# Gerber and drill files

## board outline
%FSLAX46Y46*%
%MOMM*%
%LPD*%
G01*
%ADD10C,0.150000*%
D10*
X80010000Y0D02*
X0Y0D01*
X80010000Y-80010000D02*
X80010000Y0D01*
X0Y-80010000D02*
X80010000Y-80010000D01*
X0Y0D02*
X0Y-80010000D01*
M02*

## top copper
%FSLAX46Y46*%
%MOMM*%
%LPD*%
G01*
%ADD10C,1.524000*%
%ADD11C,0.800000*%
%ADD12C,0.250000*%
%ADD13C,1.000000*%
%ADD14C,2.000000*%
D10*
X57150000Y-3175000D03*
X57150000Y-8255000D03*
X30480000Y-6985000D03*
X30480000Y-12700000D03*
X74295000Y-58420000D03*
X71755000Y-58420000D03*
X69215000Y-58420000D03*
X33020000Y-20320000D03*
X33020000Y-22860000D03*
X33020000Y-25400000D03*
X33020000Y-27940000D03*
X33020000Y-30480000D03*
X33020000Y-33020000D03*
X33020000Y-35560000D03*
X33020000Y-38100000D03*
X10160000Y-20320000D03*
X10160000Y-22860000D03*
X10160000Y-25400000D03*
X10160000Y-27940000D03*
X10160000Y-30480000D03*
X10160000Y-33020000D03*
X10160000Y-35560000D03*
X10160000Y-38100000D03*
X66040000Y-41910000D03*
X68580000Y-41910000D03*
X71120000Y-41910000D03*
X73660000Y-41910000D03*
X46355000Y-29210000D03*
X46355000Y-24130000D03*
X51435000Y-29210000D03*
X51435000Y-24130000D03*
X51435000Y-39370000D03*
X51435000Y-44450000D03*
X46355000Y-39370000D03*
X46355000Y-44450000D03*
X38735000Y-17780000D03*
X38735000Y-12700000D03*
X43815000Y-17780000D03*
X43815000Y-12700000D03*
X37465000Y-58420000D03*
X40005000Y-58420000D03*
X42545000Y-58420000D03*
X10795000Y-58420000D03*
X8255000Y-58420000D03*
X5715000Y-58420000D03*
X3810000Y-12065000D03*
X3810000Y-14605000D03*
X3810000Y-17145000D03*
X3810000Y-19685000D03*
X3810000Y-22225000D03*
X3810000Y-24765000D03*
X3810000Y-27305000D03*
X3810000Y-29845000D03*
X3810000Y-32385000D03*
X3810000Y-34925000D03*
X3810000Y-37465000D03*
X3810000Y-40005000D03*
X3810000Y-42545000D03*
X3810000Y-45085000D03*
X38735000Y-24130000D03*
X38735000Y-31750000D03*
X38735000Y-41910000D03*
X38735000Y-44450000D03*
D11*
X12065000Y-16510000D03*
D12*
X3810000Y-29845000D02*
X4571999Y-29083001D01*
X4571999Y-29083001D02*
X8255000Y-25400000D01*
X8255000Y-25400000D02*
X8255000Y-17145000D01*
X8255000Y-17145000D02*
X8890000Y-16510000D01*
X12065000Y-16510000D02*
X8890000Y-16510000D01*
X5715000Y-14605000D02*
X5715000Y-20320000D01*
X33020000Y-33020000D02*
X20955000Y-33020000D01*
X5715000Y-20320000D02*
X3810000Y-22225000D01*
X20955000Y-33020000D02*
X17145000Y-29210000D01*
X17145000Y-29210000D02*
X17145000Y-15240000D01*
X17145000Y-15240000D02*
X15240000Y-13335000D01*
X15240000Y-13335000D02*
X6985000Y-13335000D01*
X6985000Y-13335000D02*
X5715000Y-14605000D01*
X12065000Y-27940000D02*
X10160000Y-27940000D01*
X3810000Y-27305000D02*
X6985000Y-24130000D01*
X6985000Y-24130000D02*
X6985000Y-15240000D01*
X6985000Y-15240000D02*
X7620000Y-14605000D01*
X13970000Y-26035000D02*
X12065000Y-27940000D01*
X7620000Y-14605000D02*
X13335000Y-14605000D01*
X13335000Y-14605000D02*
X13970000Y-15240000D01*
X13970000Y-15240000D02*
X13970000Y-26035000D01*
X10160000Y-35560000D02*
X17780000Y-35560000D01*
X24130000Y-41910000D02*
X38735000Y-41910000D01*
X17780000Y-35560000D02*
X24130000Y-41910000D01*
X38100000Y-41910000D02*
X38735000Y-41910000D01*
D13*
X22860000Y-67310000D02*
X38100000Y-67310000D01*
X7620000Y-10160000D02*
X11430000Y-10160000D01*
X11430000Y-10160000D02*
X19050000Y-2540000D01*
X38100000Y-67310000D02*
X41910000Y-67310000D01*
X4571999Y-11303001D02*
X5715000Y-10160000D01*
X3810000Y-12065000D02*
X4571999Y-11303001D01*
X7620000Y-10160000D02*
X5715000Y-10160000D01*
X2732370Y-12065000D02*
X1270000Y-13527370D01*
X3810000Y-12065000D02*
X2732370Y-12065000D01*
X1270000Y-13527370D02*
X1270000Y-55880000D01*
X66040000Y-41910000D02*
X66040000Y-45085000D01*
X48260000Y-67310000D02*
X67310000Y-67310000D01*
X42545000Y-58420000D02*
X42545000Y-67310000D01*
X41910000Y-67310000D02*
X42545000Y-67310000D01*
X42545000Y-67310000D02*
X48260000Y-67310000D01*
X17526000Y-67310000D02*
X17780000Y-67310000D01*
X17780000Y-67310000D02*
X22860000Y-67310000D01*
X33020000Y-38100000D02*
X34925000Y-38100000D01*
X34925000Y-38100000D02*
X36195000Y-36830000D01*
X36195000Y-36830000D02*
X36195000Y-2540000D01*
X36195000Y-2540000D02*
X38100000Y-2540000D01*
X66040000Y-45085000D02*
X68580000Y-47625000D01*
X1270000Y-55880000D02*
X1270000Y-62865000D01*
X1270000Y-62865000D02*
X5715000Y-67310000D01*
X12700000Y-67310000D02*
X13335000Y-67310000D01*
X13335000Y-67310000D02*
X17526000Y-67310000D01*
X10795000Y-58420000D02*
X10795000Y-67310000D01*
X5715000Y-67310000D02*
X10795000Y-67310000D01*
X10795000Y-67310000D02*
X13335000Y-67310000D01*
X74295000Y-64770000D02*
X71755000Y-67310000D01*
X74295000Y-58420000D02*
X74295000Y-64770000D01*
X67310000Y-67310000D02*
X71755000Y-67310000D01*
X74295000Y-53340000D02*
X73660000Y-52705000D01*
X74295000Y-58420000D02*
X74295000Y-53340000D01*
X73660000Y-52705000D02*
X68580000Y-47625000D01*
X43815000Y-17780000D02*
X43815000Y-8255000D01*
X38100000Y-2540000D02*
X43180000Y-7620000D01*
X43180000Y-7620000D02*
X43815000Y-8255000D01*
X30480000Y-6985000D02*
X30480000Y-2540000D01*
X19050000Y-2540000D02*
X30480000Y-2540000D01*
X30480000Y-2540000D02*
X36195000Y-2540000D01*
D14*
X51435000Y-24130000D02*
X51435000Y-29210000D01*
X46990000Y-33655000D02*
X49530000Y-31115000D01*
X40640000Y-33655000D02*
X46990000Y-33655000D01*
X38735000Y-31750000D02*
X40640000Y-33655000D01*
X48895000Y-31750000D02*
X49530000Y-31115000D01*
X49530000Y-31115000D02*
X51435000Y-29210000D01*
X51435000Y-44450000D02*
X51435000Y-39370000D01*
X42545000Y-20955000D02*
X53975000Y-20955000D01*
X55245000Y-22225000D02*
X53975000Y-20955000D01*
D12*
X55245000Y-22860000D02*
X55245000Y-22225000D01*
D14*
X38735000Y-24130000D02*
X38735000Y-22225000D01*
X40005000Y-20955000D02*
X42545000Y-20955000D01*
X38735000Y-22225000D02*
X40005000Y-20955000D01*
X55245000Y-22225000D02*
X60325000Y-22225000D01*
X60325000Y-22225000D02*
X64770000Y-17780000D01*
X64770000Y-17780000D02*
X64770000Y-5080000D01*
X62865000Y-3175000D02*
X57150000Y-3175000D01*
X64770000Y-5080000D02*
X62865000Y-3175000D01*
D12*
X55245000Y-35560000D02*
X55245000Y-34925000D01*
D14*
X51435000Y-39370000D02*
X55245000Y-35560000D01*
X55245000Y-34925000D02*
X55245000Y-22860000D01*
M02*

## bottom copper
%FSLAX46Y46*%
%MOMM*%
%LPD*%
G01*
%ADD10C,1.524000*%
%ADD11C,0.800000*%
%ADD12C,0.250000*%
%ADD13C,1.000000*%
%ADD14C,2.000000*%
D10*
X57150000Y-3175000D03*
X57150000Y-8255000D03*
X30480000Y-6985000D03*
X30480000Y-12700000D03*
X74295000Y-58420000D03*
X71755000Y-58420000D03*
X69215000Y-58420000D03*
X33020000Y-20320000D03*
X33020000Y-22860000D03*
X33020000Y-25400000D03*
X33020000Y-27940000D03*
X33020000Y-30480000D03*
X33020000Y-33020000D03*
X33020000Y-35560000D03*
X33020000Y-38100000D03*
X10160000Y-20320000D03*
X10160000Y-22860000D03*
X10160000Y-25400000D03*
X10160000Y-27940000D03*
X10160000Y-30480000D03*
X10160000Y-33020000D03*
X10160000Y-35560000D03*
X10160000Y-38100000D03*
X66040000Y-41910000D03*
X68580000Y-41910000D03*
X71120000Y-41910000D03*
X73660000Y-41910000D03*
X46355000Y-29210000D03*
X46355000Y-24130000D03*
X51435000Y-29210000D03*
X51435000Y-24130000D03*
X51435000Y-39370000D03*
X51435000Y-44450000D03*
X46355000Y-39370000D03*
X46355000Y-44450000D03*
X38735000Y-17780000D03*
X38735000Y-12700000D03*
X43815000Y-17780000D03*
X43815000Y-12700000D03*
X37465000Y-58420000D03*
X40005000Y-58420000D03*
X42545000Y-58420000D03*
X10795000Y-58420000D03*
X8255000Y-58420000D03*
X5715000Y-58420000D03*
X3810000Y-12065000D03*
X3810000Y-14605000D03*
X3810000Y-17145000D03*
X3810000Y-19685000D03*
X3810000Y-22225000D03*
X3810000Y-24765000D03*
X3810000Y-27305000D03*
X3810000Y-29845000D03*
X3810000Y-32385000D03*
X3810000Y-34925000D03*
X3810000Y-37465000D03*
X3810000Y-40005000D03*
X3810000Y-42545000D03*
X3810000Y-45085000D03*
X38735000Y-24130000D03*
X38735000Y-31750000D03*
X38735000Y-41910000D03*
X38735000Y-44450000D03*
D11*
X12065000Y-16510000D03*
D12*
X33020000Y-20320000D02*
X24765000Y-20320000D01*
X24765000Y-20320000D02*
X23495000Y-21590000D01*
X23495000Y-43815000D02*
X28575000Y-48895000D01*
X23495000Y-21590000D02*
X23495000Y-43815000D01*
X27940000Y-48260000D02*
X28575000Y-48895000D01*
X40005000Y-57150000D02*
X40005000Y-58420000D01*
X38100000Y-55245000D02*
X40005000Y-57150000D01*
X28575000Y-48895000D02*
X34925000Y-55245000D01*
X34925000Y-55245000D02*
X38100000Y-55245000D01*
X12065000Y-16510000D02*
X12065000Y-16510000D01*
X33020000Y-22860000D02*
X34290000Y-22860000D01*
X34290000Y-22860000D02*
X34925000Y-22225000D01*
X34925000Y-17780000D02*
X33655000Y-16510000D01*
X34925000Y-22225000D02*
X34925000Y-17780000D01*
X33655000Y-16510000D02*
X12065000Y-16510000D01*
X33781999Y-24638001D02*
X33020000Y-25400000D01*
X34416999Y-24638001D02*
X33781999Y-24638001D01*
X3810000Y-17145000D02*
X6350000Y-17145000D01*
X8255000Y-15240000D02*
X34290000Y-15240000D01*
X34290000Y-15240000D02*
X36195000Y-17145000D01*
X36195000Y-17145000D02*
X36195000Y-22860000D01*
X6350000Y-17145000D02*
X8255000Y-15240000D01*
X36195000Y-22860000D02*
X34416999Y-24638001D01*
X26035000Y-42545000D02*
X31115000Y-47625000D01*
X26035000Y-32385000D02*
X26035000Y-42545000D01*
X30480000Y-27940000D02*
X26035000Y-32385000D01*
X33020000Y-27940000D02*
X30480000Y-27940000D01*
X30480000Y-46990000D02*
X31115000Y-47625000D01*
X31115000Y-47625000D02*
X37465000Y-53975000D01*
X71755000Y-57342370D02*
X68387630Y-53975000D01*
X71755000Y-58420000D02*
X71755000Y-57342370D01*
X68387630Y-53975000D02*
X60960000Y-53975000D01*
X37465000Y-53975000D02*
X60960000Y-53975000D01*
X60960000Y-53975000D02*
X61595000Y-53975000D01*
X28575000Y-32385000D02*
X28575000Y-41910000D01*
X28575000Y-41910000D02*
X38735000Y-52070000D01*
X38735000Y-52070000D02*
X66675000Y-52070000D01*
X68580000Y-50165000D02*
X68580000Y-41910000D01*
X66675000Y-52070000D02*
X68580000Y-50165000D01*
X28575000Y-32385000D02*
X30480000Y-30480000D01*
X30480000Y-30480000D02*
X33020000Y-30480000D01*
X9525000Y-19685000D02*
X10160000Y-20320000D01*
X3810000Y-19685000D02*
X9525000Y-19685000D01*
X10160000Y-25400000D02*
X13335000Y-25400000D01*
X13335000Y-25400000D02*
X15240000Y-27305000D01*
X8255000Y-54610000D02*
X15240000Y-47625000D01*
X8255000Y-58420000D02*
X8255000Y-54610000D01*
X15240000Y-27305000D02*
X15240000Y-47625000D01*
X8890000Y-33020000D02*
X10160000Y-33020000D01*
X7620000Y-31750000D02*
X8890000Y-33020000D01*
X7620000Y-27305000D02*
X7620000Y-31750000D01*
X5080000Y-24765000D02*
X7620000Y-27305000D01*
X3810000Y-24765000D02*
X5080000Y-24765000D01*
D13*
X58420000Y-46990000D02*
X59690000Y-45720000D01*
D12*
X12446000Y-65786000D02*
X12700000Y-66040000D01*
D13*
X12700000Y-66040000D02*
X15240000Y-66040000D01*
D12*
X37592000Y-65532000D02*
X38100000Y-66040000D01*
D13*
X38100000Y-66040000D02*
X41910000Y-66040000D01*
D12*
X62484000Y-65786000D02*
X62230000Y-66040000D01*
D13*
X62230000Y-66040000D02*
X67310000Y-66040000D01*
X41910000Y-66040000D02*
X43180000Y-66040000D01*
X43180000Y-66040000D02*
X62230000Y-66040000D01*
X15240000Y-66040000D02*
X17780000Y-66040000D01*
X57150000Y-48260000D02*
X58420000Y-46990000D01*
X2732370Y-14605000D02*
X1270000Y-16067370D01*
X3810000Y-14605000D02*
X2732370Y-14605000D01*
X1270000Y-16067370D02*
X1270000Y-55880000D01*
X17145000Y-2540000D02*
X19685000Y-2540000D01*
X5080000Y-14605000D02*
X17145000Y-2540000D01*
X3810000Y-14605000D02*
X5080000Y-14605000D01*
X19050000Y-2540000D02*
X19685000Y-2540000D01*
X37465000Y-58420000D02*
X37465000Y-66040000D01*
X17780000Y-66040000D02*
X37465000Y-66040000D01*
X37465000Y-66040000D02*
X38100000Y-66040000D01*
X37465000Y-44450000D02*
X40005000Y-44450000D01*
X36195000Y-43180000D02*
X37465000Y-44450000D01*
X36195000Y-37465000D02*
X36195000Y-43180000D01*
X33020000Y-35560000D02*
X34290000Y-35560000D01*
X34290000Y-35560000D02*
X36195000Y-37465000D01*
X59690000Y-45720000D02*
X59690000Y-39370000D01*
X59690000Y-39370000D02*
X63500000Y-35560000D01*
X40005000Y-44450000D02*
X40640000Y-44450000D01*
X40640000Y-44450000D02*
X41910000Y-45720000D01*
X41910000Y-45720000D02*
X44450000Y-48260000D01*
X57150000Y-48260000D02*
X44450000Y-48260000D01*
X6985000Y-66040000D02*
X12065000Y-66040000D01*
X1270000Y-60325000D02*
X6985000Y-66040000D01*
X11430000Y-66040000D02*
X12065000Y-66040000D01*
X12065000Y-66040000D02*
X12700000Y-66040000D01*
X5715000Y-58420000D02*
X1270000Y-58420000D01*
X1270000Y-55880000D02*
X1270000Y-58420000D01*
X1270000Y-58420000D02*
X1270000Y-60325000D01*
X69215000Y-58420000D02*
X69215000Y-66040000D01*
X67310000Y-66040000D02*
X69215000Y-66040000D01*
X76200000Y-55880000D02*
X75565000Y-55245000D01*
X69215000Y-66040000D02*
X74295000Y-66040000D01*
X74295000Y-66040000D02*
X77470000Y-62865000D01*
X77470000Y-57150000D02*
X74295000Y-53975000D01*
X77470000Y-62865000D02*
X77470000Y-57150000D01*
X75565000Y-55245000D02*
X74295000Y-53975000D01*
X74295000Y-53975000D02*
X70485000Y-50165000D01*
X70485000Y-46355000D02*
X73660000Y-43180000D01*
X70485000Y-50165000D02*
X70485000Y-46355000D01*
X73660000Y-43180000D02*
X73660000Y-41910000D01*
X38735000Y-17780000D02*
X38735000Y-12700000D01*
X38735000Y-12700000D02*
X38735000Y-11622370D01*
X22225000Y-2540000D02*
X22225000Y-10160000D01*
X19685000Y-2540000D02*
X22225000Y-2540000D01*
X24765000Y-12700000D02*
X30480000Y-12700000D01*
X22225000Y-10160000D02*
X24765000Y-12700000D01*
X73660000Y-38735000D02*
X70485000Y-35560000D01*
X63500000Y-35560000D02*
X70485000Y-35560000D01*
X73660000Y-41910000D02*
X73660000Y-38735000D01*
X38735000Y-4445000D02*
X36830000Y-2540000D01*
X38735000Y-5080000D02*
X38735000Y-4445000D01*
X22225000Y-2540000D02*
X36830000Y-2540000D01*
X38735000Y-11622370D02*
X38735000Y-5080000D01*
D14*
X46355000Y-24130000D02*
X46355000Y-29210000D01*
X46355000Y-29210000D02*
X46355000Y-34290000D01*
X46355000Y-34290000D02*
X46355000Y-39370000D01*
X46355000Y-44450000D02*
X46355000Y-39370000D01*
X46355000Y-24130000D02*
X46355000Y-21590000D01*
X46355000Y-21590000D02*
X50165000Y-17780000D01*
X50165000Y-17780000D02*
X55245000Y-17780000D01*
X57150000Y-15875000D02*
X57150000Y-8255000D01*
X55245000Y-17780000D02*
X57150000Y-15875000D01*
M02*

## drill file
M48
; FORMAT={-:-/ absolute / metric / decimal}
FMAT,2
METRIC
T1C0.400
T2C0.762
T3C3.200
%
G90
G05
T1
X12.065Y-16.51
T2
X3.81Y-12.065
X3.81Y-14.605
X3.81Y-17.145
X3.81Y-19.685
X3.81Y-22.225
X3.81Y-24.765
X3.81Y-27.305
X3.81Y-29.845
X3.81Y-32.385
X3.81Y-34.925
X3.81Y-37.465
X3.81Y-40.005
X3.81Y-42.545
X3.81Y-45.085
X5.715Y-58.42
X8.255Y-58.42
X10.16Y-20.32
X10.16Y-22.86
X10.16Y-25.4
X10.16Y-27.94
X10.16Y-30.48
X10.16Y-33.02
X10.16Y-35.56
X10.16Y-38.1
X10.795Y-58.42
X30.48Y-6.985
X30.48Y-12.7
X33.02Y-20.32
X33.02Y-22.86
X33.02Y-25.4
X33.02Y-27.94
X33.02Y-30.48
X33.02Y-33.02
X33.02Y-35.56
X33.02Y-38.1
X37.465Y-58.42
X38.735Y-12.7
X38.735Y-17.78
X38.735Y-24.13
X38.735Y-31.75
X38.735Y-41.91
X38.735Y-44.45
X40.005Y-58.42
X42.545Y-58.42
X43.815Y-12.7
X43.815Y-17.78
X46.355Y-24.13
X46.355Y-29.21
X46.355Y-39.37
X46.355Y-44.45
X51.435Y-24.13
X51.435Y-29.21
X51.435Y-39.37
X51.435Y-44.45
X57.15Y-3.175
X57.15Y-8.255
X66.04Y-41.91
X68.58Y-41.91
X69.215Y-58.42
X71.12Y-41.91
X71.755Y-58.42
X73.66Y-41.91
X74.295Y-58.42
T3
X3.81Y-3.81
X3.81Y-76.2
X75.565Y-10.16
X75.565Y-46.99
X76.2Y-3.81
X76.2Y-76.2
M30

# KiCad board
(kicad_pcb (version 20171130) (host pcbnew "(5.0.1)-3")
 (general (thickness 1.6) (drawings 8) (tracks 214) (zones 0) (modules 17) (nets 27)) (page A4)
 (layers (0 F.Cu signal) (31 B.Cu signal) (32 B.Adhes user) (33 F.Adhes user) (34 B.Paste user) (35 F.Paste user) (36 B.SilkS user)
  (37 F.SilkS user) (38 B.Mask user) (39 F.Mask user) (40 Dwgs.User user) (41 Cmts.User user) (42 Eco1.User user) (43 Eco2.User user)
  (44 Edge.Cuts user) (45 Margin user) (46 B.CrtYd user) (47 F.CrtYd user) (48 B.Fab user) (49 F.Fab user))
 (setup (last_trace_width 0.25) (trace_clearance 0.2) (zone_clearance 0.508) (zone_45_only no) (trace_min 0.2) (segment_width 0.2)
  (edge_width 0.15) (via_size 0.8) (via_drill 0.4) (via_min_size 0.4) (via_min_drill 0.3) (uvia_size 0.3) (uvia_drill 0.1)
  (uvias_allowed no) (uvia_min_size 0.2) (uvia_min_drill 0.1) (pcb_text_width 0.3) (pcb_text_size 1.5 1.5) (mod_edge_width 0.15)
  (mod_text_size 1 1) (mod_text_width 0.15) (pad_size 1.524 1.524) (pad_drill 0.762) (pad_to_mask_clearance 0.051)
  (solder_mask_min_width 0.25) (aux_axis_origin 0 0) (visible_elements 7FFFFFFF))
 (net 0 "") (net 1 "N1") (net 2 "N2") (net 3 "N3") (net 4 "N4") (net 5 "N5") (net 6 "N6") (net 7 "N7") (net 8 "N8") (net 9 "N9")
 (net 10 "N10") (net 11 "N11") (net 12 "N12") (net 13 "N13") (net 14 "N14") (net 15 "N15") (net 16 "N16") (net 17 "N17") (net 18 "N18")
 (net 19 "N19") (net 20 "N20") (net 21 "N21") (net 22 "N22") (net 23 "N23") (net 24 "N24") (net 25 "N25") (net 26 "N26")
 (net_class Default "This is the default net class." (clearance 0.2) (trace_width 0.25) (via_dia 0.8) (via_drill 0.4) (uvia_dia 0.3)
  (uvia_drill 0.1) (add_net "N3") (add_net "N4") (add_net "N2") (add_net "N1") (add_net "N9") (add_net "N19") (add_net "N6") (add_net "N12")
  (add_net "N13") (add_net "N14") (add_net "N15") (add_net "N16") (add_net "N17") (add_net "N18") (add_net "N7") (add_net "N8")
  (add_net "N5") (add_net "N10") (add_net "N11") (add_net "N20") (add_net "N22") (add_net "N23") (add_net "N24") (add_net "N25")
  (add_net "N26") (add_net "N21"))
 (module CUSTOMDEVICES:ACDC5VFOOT (layer F.Cu) (at 58.42 0 270)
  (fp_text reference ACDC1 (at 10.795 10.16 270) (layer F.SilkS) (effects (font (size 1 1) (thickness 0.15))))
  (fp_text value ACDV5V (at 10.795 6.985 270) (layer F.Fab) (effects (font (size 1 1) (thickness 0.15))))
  (pad 2 thru_hole circle (at 3.175 1.27 270) (size 1.524 1.524) (drill 0.762) (layers *.Cu *.Mask) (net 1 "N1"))
  (pad 1 thru_hole circle (at 8.255 1.27 270) (size 1.524 1.524) (drill 0.762) (layers *.Cu *.Mask) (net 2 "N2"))
  (pad 4 thru_hole circle (at 6.985 27.94 270) (size 1.524 1.524) (drill 0.762) (layers *.Cu *.Mask) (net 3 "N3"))
  (pad 3 thru_hole circle (at 12.7 27.94 270) (size 1.524 1.524) (drill 0.762) (layers *.Cu *.Mask) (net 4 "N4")))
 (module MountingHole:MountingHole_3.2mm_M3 (layer F.Cu) (at 75.565 46.99)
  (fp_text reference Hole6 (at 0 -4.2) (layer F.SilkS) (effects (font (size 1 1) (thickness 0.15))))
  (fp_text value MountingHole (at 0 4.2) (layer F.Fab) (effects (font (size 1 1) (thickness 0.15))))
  (pad 1 np_thru_hole circle (at 0 0) (size 3.2 3.2) (drill 3.2) (layers *.Cu *.Mask)))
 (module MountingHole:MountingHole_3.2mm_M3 (layer F.Cu) (at 75.565 10.16)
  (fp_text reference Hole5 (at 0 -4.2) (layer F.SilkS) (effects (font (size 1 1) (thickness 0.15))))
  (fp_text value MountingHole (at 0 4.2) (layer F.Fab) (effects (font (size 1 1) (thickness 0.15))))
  (pad 1 np_thru_hole circle (at 0 0) (size 3.2 3.2) (drill 3.2) (layers *.Cu *.Mask)))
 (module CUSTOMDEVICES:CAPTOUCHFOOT (layer F.Cu) (at 71.755 63.5 180)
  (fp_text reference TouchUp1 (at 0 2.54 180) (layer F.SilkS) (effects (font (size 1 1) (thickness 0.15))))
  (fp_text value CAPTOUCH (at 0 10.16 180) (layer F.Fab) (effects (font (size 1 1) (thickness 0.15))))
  (pad 1 thru_hole circle (at -2.54 5.08 180) (size 1.524 1.524) (drill 0.762) (layers *.Cu *.Mask) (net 3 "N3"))
  (pad 2 thru_hole circle (at 0 5.08 180) (size 1.524 1.524) (drill 0.762) (layers *.Cu *.Mask) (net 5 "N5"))
  (pad 3 thru_hole circle (at 2.54 5.08 180) (size 1.524 1.524) (drill 0.762) (layers *.Cu *.Mask) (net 4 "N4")))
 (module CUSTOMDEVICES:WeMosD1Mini (layer F.Cu) (at 21.59 30.48)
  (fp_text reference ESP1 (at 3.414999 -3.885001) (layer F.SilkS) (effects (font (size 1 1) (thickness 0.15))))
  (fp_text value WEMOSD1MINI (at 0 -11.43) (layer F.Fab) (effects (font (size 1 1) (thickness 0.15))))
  (pad 1 thru_hole circle (at 11.43 -10.16) (size 1.524 1.524) (drill 0.762) (layers *.Cu *.Mask) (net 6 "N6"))
  (pad 2 thru_hole circle (at 11.43 -7.62) (size 1.524 1.524) (drill 0.762) (layers *.Cu *.Mask) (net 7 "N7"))
  (pad 3 thru_hole circle (at 11.43 -5.08) (size 1.524 1.524) (drill 0.762) (layers *.Cu *.Mask) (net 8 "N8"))
  (pad 4 thru_hole circle (at 11.43 -2.54) (size 1.524 1.524) (drill 0.762) (layers *.Cu *.Mask) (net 5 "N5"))
  (pad 5 thru_hole circle (at 11.43 0) (size 1.524 1.524) (drill 0.762) (layers *.Cu *.Mask) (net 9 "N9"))
  (pad 6 thru_hole circle (at 11.43 2.54) (size 1.524 1.524) (drill 0.762) (layers *.Cu *.Mask) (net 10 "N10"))
  (pad 7 thru_hole circle (at 11.43 5.08) (size 1.524 1.524) (drill 0.762) (layers *.Cu *.Mask) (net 4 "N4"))
  (pad 8 thru_hole circle (at 11.43 7.62) (size 1.524 1.524) (drill 0.762) (layers *.Cu *.Mask) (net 3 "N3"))
  (pad 9 thru_hole circle (at -11.43 -10.16) (size 1.524 1.524) (drill 0.762) (layers *.Cu *.Mask) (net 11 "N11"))
  (pad 10 thru_hole circle (at -11.43 -7.62) (size 1.524 1.524) (drill 0.762) (layers *.Cu *.Mask) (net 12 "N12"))
  (pad 11 thru_hole circle (at -11.43 -5.08) (size 1.524 1.524) (drill 0.762) (layers *.Cu *.Mask) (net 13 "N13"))
  (pad 12 thru_hole circle (at -11.43 -2.54) (size 1.524 1.524) (drill 0.762) (layers *.Cu *.Mask) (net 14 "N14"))
  (pad 13 thru_hole circle (at -11.43 0) (size 1.524 1.524) (drill 0.762) (layers *.Cu *.Mask) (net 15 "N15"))
  (pad 14 thru_hole circle (at -11.43 2.54) (size 1.524 1.524) (drill 0.762) (layers *.Cu *.Mask) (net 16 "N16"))
  (pad 15 thru_hole circle (at -11.43 5.08) (size 1.524 1.524) (drill 0.762) (layers *.Cu *.Mask) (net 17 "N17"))
  (pad 16 thru_hole circle (at -11.43 7.62) (size 1.524 1.524) (drill 0.762) (layers *.Cu *.Mask) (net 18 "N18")))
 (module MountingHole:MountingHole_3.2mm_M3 (layer F.Cu) (at 76.2 76.2)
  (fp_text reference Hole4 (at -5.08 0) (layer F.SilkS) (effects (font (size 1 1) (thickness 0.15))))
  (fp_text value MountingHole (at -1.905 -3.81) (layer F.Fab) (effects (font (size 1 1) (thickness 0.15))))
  (pad 1 np_thru_hole circle (at 0 0) (size 3.2 3.2) (drill 3.2) (layers *.Cu *.Mask)))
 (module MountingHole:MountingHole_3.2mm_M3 (layer F.Cu) (at 3.81 76.2)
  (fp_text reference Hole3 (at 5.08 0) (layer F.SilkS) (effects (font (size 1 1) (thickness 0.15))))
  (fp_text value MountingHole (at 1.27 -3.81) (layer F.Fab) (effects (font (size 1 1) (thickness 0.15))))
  (pad 1 np_thru_hole circle (at 0 0) (size 3.2 3.2) (drill 3.2) (layers *.Cu *.Mask)))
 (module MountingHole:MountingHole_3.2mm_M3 (layer F.Cu) (at 76.2 3.81)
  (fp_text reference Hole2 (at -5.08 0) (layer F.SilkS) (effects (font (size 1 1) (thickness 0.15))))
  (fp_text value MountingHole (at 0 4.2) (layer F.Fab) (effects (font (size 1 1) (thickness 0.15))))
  (pad 1 np_thru_hole circle (at 0 0) (size 3.2 3.2) (drill 3.2) (layers *.Cu *.Mask)))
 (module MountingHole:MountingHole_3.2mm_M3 (layer F.Cu) (at 3.81 3.81)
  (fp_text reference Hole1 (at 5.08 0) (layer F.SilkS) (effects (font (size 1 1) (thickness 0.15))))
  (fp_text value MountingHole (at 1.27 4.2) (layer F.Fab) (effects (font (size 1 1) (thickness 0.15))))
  (pad 1 np_thru_hole circle (at 0 0) (size 3.2 3.2) (drill 3.2) (layers *.Cu *.Mask)))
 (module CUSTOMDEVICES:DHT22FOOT (layer F.Cu) (at 71.12 29.21)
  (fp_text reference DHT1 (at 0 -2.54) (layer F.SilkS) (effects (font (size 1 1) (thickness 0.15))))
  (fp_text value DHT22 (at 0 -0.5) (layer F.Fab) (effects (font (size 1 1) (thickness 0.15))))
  (pad 1 thru_hole circle (at -5.08 12.7) (size 1.524 1.524) (drill 0.762) (layers *.Cu *.Mask) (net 3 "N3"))
  (pad 2 thru_hole circle (at -2.54 12.7) (size 1.524 1.524) (drill 0.762) (layers *.Cu *.Mask) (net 9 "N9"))
  (pad 3 thru_hole circle (at 0 12.7) (size 1.524 1.524) (drill 0.762) (layers *.Cu *.Mask) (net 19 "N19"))
  (pad 4 thru_hole circle (at 2.54 12.7) (size 1.524 1.524) (drill 0.762) (layers *.Cu *.Mask) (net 4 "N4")))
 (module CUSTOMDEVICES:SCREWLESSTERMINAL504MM (layer F.Cu) (at 46.355 26.67 180)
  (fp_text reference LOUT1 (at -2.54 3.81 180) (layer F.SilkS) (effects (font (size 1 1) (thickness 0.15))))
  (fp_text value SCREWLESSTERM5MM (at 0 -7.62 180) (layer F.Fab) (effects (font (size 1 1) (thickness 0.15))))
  (pad 2 thru_hole circle (at 0 -2.54 180) (size 1.524 1.524) (drill 0.762) (layers *.Cu *.Mask) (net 2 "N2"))
  (pad 2 thru_hole circle (at 0 2.54 180) (size 1.524 1.524) (drill 0.762) (layers *.Cu *.Mask) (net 2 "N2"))
  (pad 1 thru_hole circle (at -5.08 -2.54 180) (size 1.524 1.524) (drill 0.762) (layers *.Cu *.Mask) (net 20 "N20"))
  (pad 1 thru_hole circle (at -5.08 2.54 180) (size 1.524 1.524) (drill 0.762) (layers *.Cu *.Mask) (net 20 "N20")))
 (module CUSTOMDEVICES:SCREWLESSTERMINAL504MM (layer F.Cu) (at 46.355 41.91 180)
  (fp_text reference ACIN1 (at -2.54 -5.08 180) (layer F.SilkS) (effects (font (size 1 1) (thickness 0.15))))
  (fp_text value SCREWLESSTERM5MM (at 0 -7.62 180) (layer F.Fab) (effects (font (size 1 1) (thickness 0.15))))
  (pad 1 thru_hole circle (at -5.08 2.54 180) (size 1.524 1.524) (drill 0.762) (layers *.Cu *.Mask) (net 1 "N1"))
  (pad 1 thru_hole circle (at -5.08 -2.54 180) (size 1.524 1.524) (drill 0.762) (layers *.Cu *.Mask) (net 1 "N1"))
  (pad 2 thru_hole circle (at 0 2.54 180) (size 1.524 1.524) (drill 0.762) (layers *.Cu *.Mask) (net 2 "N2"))
  (pad 2 thru_hole circle (at 0 -2.54 180) (size 1.524 1.524) (drill 0.762) (layers *.Cu *.Mask) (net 2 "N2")))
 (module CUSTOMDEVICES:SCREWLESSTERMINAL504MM (layer F.Cu) (at 38.735 15.24 180)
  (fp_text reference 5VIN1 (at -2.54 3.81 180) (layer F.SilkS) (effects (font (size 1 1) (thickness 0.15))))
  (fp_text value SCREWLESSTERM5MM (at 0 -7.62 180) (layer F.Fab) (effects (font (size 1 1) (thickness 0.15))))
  (pad 2 thru_hole circle (at 0 -2.54 180) (size 1.524 1.524) (drill 0.762) (layers *.Cu *.Mask) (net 4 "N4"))
  (pad 2 thru_hole circle (at 0 2.54 180) (size 1.524 1.524) (drill 0.762) (layers *.Cu *.Mask) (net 4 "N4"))
  (pad 1 thru_hole circle (at -5.08 -2.54 180) (size 1.524 1.524) (drill 0.762) (layers *.Cu *.Mask) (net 3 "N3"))
  (pad 1 thru_hole circle (at -5.08 2.54 180) (size 1.524 1.524) (drill 0.762) (layers *.Cu *.Mask) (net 3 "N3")))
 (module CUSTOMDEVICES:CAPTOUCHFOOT (layer F.Cu) (at 40.005 63.5 180)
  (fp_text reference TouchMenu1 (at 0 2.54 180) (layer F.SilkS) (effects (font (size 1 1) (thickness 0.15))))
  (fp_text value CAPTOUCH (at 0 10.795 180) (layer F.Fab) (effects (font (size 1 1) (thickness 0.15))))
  (pad 3 thru_hole circle (at 2.54 5.08 180) (size 1.524 1.524) (drill 0.762) (layers *.Cu *.Mask) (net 4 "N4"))
  (pad 2 thru_hole circle (at 0 5.08 180) (size 1.524 1.524) (drill 0.762) (layers *.Cu *.Mask) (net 6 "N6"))
  (pad 1 thru_hole circle (at -2.54 5.08 180) (size 1.524 1.524) (drill 0.762) (layers *.Cu *.Mask) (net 3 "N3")))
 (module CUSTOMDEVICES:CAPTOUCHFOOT (layer F.Cu) (at 8.255 63.5 180)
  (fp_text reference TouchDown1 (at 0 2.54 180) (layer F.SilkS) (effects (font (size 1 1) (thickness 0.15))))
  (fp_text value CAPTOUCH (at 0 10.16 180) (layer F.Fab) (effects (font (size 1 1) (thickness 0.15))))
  (pad 1 thru_hole circle (at -2.54 5.08 180) (size 1.524 1.524) (drill 0.762) (layers *.Cu *.Mask) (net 3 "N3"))
  (pad 2 thru_hole circle (at 0 5.08 180) (size 1.524 1.524) (drill 0.762) (layers *.Cu *.Mask) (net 13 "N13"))
  (pad 3 thru_hole circle (at 2.54 5.08 180) (size 1.524 1.524) (drill 0.762) (layers *.Cu *.Mask) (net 4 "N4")))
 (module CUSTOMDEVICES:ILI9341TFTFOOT (layer F.Cu) (at 6.35 29.845 180)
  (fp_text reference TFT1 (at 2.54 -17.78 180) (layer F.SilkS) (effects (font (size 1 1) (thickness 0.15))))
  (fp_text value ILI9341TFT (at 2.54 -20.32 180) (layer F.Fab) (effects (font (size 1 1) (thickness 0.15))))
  (pad 1 thru_hole circle (at 2.54 17.78 180) (size 1.524 1.524) (drill 0.762) (layers *.Cu *.Mask) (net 3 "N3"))
  (pad 2 thru_hole circle (at 2.54 15.24 180) (size 1.524 1.524) (drill 0.762) (layers *.Cu *.Mask) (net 4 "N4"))
  (pad 3 thru_hole circle (at 2.54 12.7 180) (size 1.524 1.524) (drill 0.762) (layers *.Cu *.Mask) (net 8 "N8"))
  (pad 4 thru_hole circle (at 2.54 10.16 180) (size 1.524 1.524) (drill 0.762) (layers *.Cu *.Mask) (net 11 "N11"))
  (pad 5 thru_hole circle (at 2.54 7.62 180) (size 1.524 1.524) (drill 0.762) (layers *.Cu *.Mask) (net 10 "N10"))
  (pad 6 thru_hole circle (at 2.54 5.08 180) (size 1.524 1.524) (drill 0.762) (layers *.Cu *.Mask) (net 16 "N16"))
  (pad 7 thru_hole circle (at 2.54 2.54 180) (size 1.524 1.524) (drill 0.762) (layers *.Cu *.Mask) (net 14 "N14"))
  (pad 8 thru_hole circle (at 2.54 0 180) (size 1.524 1.524) (drill 0.762) (layers *.Cu *.Mask) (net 7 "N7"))
  (pad 9 thru_hole circle (at 2.54 -2.54 180) (size 1.524 1.524) (drill 0.762) (layers *.Cu *.Mask) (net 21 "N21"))
  (pad 10 thru_hole circle (at 2.54 -5.08 180) (size 1.524 1.524) (drill 0.762) (layers *.Cu *.Mask) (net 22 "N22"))
  (pad 11 thru_hole circle (at 2.54 -7.62 180) (size 1.524 1.524) (drill 0.762) (layers *.Cu *.Mask) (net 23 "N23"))
  (pad 12 thru_hole circle (at 2.54 -10.16 180) (size 1.524 1.524) (drill 0.762) (layers *.Cu *.Mask) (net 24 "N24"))
  (pad 13 thru_hole circle (at 2.54 -12.7 180) (size 1.524 1.524) (drill 0.762) (layers *.Cu *.Mask) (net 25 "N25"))
  (pad 14 thru_hole circle (at 2.54 -15.24 180) (size 1.524 1.524) (drill 0.762) (layers *.Cu *.Mask) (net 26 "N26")))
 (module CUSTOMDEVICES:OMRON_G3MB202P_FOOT (layer F.Cu) (at 38.735 34.29)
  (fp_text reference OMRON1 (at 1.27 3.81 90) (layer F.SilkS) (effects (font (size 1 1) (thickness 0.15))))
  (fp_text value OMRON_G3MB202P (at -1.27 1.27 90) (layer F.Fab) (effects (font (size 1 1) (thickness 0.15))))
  (pad 1 thru_hole circle (at 0 -10.16) (size 1.524 1.524) (drill 0.762) (layers *.Cu *.Mask) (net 1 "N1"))
  (pad 2 thru_hole circle (at 0 -2.54) (size 1.524 1.524) (drill 0.762) (layers *.Cu *.Mask) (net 20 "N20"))
  (pad 3 thru_hole circle (at 0 7.62) (size 1.524 1.524) (drill 0.762) (layers *.Cu *.Mask) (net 17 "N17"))
  (pad 4 thru_hole circle (at 0 10.16) (size 1.524 1.524) (drill 0.762) (layers *.Cu *.Mask) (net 4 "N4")))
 (gr_line (start 80.01 0) (end 0 0) (layer Edge.Cuts) (width 0.15))
 (gr_line (start 80.01 80.01) (end 80.01 0) (layer Edge.Cuts) (width 0.15))
 (gr_line (start 0 80.01) (end 80.01 80.01) (layer Edge.Cuts) (width 0.15))
 (gr_line (start 0 0) (end 0 80.01) (layer Edge.Cuts) (width 0.15))
 (segment (start 33.02 20.32) (end 24.765 20.32) (width 0.25) (layer B.Cu) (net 6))
 (segment (start 24.765 20.32) (end 23.495 21.59) (width 0.25) (layer B.Cu) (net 6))
 (segment (start 23.495 43.815) (end 28.575 48.895) (width 0.25) (layer B.Cu) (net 6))
 (segment (start 23.495 21.59) (end 23.495 43.815) (width 0.25) (layer B.Cu) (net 6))
 (segment (start 27.94 48.26) (end 28.575 48.895) (width 0.25) (layer B.Cu) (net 6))
 (segment (start 40.005 57.15) (end 40.005 58.42) (width 0.25) (layer B.Cu) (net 6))
 (segment (start 38.1 55.245) (end 40.005 57.15) (width 0.25) (layer B.Cu) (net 6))
 (segment (start 28.575 48.895) (end 34.925 55.245) (width 0.25) (layer B.Cu) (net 6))
 (segment (start 34.925 55.245) (end 38.1 55.245) (width 0.25) (layer B.Cu) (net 6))
 (segment (start 3.81 29.845) (end 4.571999 29.083001) (width 0.25) (layer F.Cu) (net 7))
 (segment (start 4.571999 29.083001) (end 8.255 25.4) (width 0.25) (layer F.Cu) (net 7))
 (segment (start 8.255 25.4) (end 8.255 17.145) (width 0.25) (layer F.Cu) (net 7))
 (segment (start 8.255 17.145) (end 8.89 16.51) (width 0.25) (layer F.Cu) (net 7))
 (segment (start 12.065 16.51) (end 12.065 16.51) (width 0.25) (layer B.Cu) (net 7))
 (via (at 12.065 16.51) (size 0.8) (drill 0.4) (layers F.Cu B.Cu) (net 7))
 (segment (start 12.065 16.51) (end 8.89 16.51) (width 0.25) (layer F.Cu) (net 7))
 (segment (start 33.02 22.86) (end 34.29 22.86) (width 0.25) (layer B.Cu) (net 7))
 (segment (start 34.29 22.86) (end 34.925 22.225) (width 0.25) (layer B.Cu) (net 7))
 (segment (start 34.925 17.78) (end 33.655 16.51) (width 0.25) (layer B.Cu) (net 7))
 (segment (start 34.925 22.225) (end 34.925 17.78) (width 0.25) (layer B.Cu) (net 7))
 (segment (start 33.655 16.51) (end 12.065 16.51) (width 0.25) (layer B.Cu) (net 7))
 (segment (start 33.781999 24.638001) (end 33.02 25.4) (width 0.25) (layer B.Cu) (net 8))
 (segment (start 34.416999 24.638001) (end 33.781999 24.638001) (width 0.25) (layer B.Cu) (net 8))
 (segment (start 3.81 17.145) (end 6.35 17.145) (width 0.25) (layer B.Cu) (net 8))
 (segment (start 8.255 15.24) (end 34.29 15.24) (width 0.25) (layer B.Cu) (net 8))
 (segment (start 34.29 15.24) (end 36.195 17.145) (width 0.25) (layer B.Cu) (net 8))
 (segment (start 36.195 17.145) (end 36.195 22.86) (width 0.25) (layer B.Cu) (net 8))
 (segment (start 6.35 17.145) (end 8.255 15.24) (width 0.25) (layer B.Cu) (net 8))
 (segment (start 36.195 22.86) (end 34.416999 24.638001) (width 0.25) (layer B.Cu) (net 8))
 (segment (start 26.035 42.545) (end 31.115 47.625) (width 0.25) (layer B.Cu) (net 5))
 (segment (start 26.035 32.385) (end 26.035 42.545) (width 0.25) (layer B.Cu) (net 5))
 (segment (start 30.48 27.94) (end 26.035 32.385) (width 0.25) (layer B.Cu) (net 5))
 (segment (start 33.02 27.94) (end 30.48 27.94) (width 0.25) (layer B.Cu) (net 5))
 (segment (start 30.48 46.99) (end 31.115 47.625) (width 0.25) (layer B.Cu) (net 5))
 (segment (start 31.115 47.625) (end 37.465 53.975) (width 0.25) (layer B.Cu) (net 5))
 (segment (start 71.755 57.34237) (end 68.38763 53.975) (width 0.25) (layer B.Cu) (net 5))
 (segment (start 71.755 58.42) (end 71.755 57.34237) (width 0.25) (layer B.Cu) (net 5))
 (segment (start 68.38763 53.975) (end 60.96 53.975) (width 0.25) (layer B.Cu) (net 5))
 (segment (start 37.465 53.975) (end 60.96 53.975) (width 0.25) (layer B.Cu) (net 5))
 (segment (start 60.96 53.975) (end 61.595 53.975) (width 0.25) (layer B.Cu) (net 5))
 (segment (start 28.575 32.385) (end 28.575 41.91) (width 0.25) (layer B.Cu) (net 9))
 (segment (start 28.575 41.91) (end 38.735 52.07) (width 0.25) (layer B.Cu) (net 9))
 (segment (start 38.735 52.07) (end 66.675 52.07) (width 0.25) (layer B.Cu) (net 9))
 (segment (start 68.58 50.165) (end 68.58 41.91) (width 0.25) (layer B.Cu) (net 9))
 (segment (start 66.675 52.07) (end 68.58 50.165) (width 0.25) (layer B.Cu) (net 9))
 (segment (start 28.575 32.385) (end 30.48 30.48) (width 0.25) (layer B.Cu) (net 9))
 (segment (start 30.48 30.48) (end 33.02 30.48) (width 0.25) (layer B.Cu) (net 9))
 (segment (start 5.715 14.605) (end 5.715 20.32) (width 0.25) (layer F.Cu) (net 10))
 (segment (start 33.02 33.02) (end 20.955 33.02) (width 0.25) (layer F.Cu) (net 10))
 (segment (start 5.715 20.32) (end 3.81 22.225) (width 0.25) (layer F.Cu) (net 10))
 (segment (start 20.955 33.02) (end 17.145 29.21) (width 0.25) (layer F.Cu) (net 10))
 (segment (start 17.145 29.21) (end 17.145 15.24) (width 0.25) (layer F.Cu) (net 10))
 (segment (start 17.145 15.24) (end 15.24 13.335) (width 0.25) (layer F.Cu) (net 10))
 (segment (start 15.24 13.335) (end 6.985 13.335) (width 0.25) (layer F.Cu) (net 10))
 (segment (start 6.985 13.335) (end 5.715 14.605) (width 0.25) (layer F.Cu) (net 10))
 (segment (start 9.525 19.685) (end 10.16 20.32) (width 0.25) (layer B.Cu) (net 11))
 (segment (start 3.81 19.685) (end 9.525 19.685) (width 0.25) (layer B.Cu) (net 11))
 (segment (start 10.16 25.4) (end 13.335 25.4) (width 0.25) (layer B.Cu) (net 13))
 (segment (start 13.335 25.4) (end 15.24 27.305) (width 0.25) (layer B.Cu) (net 13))
 (segment (start 8.255 54.61) (end 15.24 47.625) (width 0.25) (layer B.Cu) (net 13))
 (segment (start 8.255 58.42) (end 8.255 54.61) (width 0.25) (layer B.Cu) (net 13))
 (segment (start 15.24 27.305) (end 15.24 47.625) (width 0.25) (layer B.Cu) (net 13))
 (segment (start 12.065 27.94) (end 10.16 27.94) (width 0.25) (layer F.Cu) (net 14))
 (segment (start 3.81 27.305) (end 6.985 24.13) (width 0.25) (layer F.Cu) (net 14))
 (segment (start 6.985 24.13) (end 6.985 15.24) (width 0.25) (layer F.Cu) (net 14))
 (segment (start 6.985 15.24) (end 7.62 14.605) (width 0.25) (layer F.Cu) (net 14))
 (segment (start 13.97 26.035) (end 12.065 27.94) (width 0.25) (layer F.Cu) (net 14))
 (segment (start 7.62 14.605) (end 13.335 14.605) (width 0.25) (layer F.Cu) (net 14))
 (segment (start 13.335 14.605) (end 13.97 15.24) (width 0.25) (layer F.Cu) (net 14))
 (segment (start 13.97 15.24) (end 13.97 26.035) (width 0.25) (layer F.Cu) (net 14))
 (segment (start 8.89 33.02) (end 10.16 33.02) (width 0.25) (layer B.Cu) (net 16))
 (segment (start 7.62 31.75) (end 8.89 33.02) (width 0.25) (layer B.Cu) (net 16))
 (segment (start 7.62 27.305) (end 7.62 31.75) (width 0.25) (layer B.Cu) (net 16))
 (segment (start 5.08 24.765) (end 7.62 27.305) (width 0.25) (layer B.Cu) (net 16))
 (segment (start 3.81 24.765) (end 5.08 24.765) (width 0.25) (layer B.Cu) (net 16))
 (segment (start 10.16 35.56) (end 17.78 35.56) (width 0.25) (layer F.Cu) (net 17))
 (segment (start 24.13 41.91) (end 38.735 41.91) (width 0.25) (layer F.Cu) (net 17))
 (segment (start 17.78 35.56) (end 24.13 41.91) (width 0.25) (layer F.Cu) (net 17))
 (segment (start 38.1 41.91) (end 38.735 41.91) (width 0.25) (layer F.Cu) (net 17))
 (segment (start 22.86 67.31) (end 38.1 67.31) (width 1) (layer F.Cu) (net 3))
 (segment (start 7.62 10.16) (end 11.43 10.16) (width 1) (layer F.Cu) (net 3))
 (segment (start 11.43 10.16) (end 19.05 2.54) (width 1) (layer F.Cu) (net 3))
 (segment (start 38.1 67.31) (end 41.91 67.31) (width 1) (layer F.Cu) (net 3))
 (segment (start 4.571999 11.303001) (end 5.715 10.16) (width 1) (layer F.Cu) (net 3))
 (segment (start 3.81 12.065) (end 4.571999 11.303001) (width 1) (layer F.Cu) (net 3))
 (segment (start 7.62 10.16) (end 5.715 10.16) (width 1) (layer F.Cu) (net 3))
 (segment (start 2.73237 12.065) (end 1.27 13.52737) (width 1) (layer F.Cu) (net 3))
 (segment (start 3.81 12.065) (end 2.73237 12.065) (width 1) (layer F.Cu) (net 3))
 (segment (start 1.27 13.52737) (end 1.27 55.88) (width 1) (layer F.Cu) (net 3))
 (segment (start 66.04 41.91) (end 66.04 45.085) (width 1) (layer F.Cu) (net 3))
 (segment (start 48.26 67.31) (end 67.31 67.31) (width 1) (layer F.Cu) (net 3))
 (segment (start 42.545 58.42) (end 42.545 67.31) (width 1) (layer F.Cu) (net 3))
 (segment (start 41.91 67.31) (end 42.545 67.31) (width 1) (layer F.Cu) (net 3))
 (segment (start 42.545 67.31) (end 48.26 67.31) (width 1) (layer F.Cu) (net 3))
 (segment (start 17.526 67.31) (end 17.78 67.31) (width 1) (layer F.Cu) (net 3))
 (segment (start 17.78 67.31) (end 22.86 67.31) (width 1) (layer F.Cu) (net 3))
 (segment (start 33.02 38.1) (end 34.925 38.1) (width 1) (layer F.Cu) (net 3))
 (segment (start 34.925 38.1) (end 36.195 36.83) (width 1) (layer F.Cu) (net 3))
 (segment (start 36.195 36.83) (end 36.195 2.54) (width 1) (layer F.Cu) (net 3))
 (segment (start 36.195 2.54) (end 38.1 2.54) (width 1) (layer F.Cu) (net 3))
 (segment (start 66.04 45.085) (end 68.58 47.625) (width 1) (layer F.Cu) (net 3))
 (segment (start 1.27 55.88) (end 1.27 62.865) (width 1) (layer F.Cu) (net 3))
 (segment (start 1.27 62.865) (end 5.715 67.31) (width 1) (layer F.Cu) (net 3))
 (segment (start 12.7 67.31) (end 13.335 67.31) (width 1) (layer F.Cu) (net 3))
 (segment (start 13.335 67.31) (end 17.526 67.31) (width 1) (layer F.Cu) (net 3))
 (segment (start 10.795 58.42) (end 10.795 67.31) (width 1) (layer F.Cu) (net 3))
 (segment (start 5.715 67.31) (end 10.795 67.31) (width 1) (layer F.Cu) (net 3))
 (segment (start 10.795 67.31) (end 13.335 67.31) (width 1) (layer F.Cu) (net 3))
 (segment (start 74.295 64.77) (end 71.755 67.31) (width 1) (layer F.Cu) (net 3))
 (segment (start 74.295 58.42) (end 74.295 64.77) (width 1) (layer F.Cu) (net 3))
 (segment (start 67.31 67.31) (end 71.755 67.31) (width 1) (layer F.Cu) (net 3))
 (segment (start 74.295 53.34) (end 73.66 52.705) (width 1) (layer F.Cu) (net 3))
 (segment (start 74.295 58.42) (end 74.295 53.34) (width 1) (layer F.Cu) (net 3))
 (segment (start 73.66 52.705) (end 68.58 47.625) (width 1) (layer F.Cu) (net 3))
 (segment (start 43.815 17.78) (end 43.815 8.255) (width 1) (layer F.Cu) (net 3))
 (segment (start 38.1 2.54) (end 43.18 7.62) (width 1) (layer F.Cu) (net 3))
 (segment (start 43.18 7.62) (end 43.815 8.255) (width 1) (layer F.Cu) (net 3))
 (segment (start 30.48 6.985) (end 30.48 2.54) (width 1) (layer F.Cu) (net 3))
 (segment (start 19.05 2.54) (end 30.48 2.54) (width 1) (layer F.Cu) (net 3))
 (segment (start 30.48 2.54) (end 36.195 2.54) (width 1) (layer F.Cu) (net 3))
 (segment (start 58.42 46.99) (end 59.69 45.72) (width 1) (layer B.Cu) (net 4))
 (segment (start 12.446 65.786) (end 12.7 66.04) (width 0.25) (layer B.Cu) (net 4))
 (segment (start 12.7 66.04) (end 15.24 66.04) (width 1) (layer B.Cu) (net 4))
 (segment (start 37.592 65.532) (end 38.1 66.04) (width 0.25) (layer B.Cu) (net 4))
 (segment (start 38.1 66.04) (end 41.91 66.04) (width 1) (layer B.Cu) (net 4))
 (segment (start 62.484 65.786) (end 62.23 66.04) (width 0.25) (layer B.Cu) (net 4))
 (segment (start 62.23 66.04) (end 67.31 66.04) (width 1) (layer B.Cu) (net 4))
 (segment (start 41.91 66.04) (end 43.18 66.04) (width 1) (layer B.Cu) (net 4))
 (segment (start 43.18 66.04) (end 62.23 66.04) (width 1) (layer B.Cu) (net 4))
 (segment (start 15.24 66.04) (end 17.78 66.04) (width 1) (layer B.Cu) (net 4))
 (segment (start 57.15 48.26) (end 58.42 46.99) (width 1) (layer B.Cu) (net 4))
 (segment (start 2.73237 14.605) (end 1.27 16.06737) (width 1) (layer B.Cu) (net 4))
 (segment (start 3.81 14.605) (end 2.73237 14.605) (width 1) (layer B.Cu) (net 4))
 (segment (start 1.27 16.06737) (end 1.27 55.88) (width 1) (layer B.Cu) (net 4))
 (segment (start 17.145 2.54) (end 19.685 2.54) (width 1) (layer B.Cu) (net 4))
 (segment (start 5.08 14.605) (end 17.145 2.54) (width 1) (layer B.Cu) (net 4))
 (segment (start 3.81 14.605) (end 5.08 14.605) (width 1) (layer B.Cu) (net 4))
 (segment (start 19.05 2.54) (end 19.685 2.54) (width 1) (layer B.Cu) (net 4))
 (segment (start 37.465 58.42) (end 37.465 66.04) (width 1) (layer B.Cu) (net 4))
 (segment (start 17.78 66.04) (end 37.465 66.04) (width 1) (layer B.Cu) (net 4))
 (segment (start 37.465 66.04) (end 38.1 66.04) (width 1) (layer B.Cu) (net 4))
 (segment (start 37.465 44.45) (end 40.005 44.45) (width 1) (layer B.Cu) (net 4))
 (segment (start 36.195 43.18) (end 37.465 44.45) (width 1) (layer B.Cu) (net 4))
 (segment (start 36.195 37.465) (end 36.195 43.18) (width 1) (layer B.Cu) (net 4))
 (segment (start 33.02 35.56) (end 34.29 35.56) (width 1) (layer B.Cu) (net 4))
 (segment (start 34.29 35.56) (end 36.195 37.465) (width 1) (layer B.Cu) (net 4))
 (segment (start 59.69 45.72) (end 59.69 39.37) (width 1) (layer B.Cu) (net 4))
 (segment (start 59.69 39.37) (end 63.5 35.56) (width 1) (layer B.Cu) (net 4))
 (segment (start 40.005 44.45) (end 40.64 44.45) (width 1) (layer B.Cu) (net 4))
 (segment (start 40.64 44.45) (end 41.91 45.72) (width 1) (layer B.Cu) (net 4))
 (segment (start 41.91 45.72) (end 44.45 48.26) (width 1) (layer B.Cu) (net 4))
 (segment (start 57.15 48.26) (end 44.45 48.26) (width 1) (layer B.Cu) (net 4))
 (segment (start 6.985 66.04) (end 12.065 66.04) (width 1) (layer B.Cu) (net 4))
 (segment (start 1.27 60.325) (end 6.985 66.04) (width 1) (layer B.Cu) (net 4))
 (segment (start 11.43 66.04) (end 12.065 66.04) (width 1) (layer B.Cu) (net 4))
 (segment (start 12.065 66.04) (end 12.7 66.04) (width 1) (layer B.Cu) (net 4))
 (segment (start 5.715 58.42) (end 1.27 58.42) (width 1) (layer B.Cu) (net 4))
 (segment (start 1.27 55.88) (end 1.27 58.42) (width 1) (layer B.Cu) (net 4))
 (segment (start 1.27 58.42) (end 1.27 60.325) (width 1) (layer B.Cu) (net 4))
 (segment (start 69.215 58.42) (end 69.215 66.04) (width 1) (layer B.Cu) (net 4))
 (segment (start 67.31 66.04) (end 69.215 66.04) (width 1) (layer B.Cu) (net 4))
 (segment (start 76.2 55.88) (end 75.565 55.245) (width 1) (layer B.Cu) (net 4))
 (segment (start 69.215 66.04) (end 74.295 66.04) (width 1) (layer B.Cu) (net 4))
 (segment (start 74.295 66.04) (end 77.47 62.865) (width 1) (layer B.Cu) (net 4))
 (segment (start 77.47 57.15) (end 74.295 53.975) (width 1) (layer B.Cu) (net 4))
 (segment (start 77.47 62.865) (end 77.47 57.15) (width 1) (layer B.Cu) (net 4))
 (segment (start 75.565 55.245) (end 74.295 53.975) (width 1) (layer B.Cu) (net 4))
 (segment (start 74.295 53.975) (end 70.485 50.165) (width 1) (layer B.Cu) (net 4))
 (segment (start 70.485 46.355) (end 73.66 43.18) (width 1) (layer B.Cu) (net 4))
 (segment (start 70.485 50.165) (end 70.485 46.355) (width 1) (layer B.Cu) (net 4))
 (segment (start 73.66 43.18) (end 73.66 41.91) (width 1) (layer B.Cu) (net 4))
 (segment (start 38.735 17.78) (end 38.735 12.7) (width 1) (layer B.Cu) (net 4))
 (segment (start 38.735 12.7) (end 38.735 11.62237) (width 1) (layer B.Cu) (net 4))
 (segment (start 22.225 2.54) (end 22.225 10.16) (width 1) (layer B.Cu) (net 4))
 (segment (start 19.685 2.54) (end 22.225 2.54) (width 1) (layer B.Cu) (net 4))
 (segment (start 24.765 12.7) (end 30.48 12.7) (width 1) (layer B.Cu) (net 4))
 (segment (start 22.225 10.16) (end 24.765 12.7) (width 1) (layer B.Cu) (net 4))
 (segment (start 73.66 38.735) (end 70.485 35.56) (width 1) (layer B.Cu) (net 4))
 (segment (start 63.5 35.56) (end 70.485 35.56) (width 1) (layer B.Cu) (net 4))
 (segment (start 73.66 41.91) (end 73.66 38.735) (width 1) (layer B.Cu) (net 4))
 (segment (start 38.735 4.445) (end 36.83 2.54) (width 1) (layer B.Cu) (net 4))
 (segment (start 38.735 5.08) (end 38.735 4.445) (width 1) (layer B.Cu) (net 4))
 (segment (start 22.225 2.54) (end 36.83 2.54) (width 1) (layer B.Cu) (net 4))
 (segment (start 38.735 11.62237) (end 38.735 5.08) (width 1) (layer B.Cu) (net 4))
 (segment (start 51.435 24.13) (end 51.435 29.21) (width 2) (layer F.Cu) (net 20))
 (segment (start 46.99 33.655) (end 49.53 31.115) (width 2) (layer F.Cu) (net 20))
 (segment (start 40.64 33.655) (end 46.99 33.655) (width 2) (layer F.Cu) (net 20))
 (segment (start 38.735 31.75) (end 40.64 33.655) (width 2) (layer F.Cu) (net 20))
 (segment (start 48.895 31.75) (end 49.53 31.115) (width 2) (layer F.Cu) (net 20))
 (segment (start 49.53 31.115) (end 51.435 29.21) (width 2) (layer F.Cu) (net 20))
 (segment (start 51.435 44.45) (end 51.435 39.37) (width 2) (layer F.Cu) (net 1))
 (segment (start 42.545 20.955) (end 53.975 20.955) (width 2) (layer F.Cu) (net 1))
 (segment (start 55.245 22.225) (end 53.975 20.955) (width 2) (layer F.Cu) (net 1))
 (segment (start 55.245 22.86) (end 55.245 22.225) (width 0.25) (layer F.Cu) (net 1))
 (segment (start 38.735 24.13) (end 38.735 22.225) (width 2) (layer F.Cu) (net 1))
 (segment (start 40.005 20.955) (end 42.545 20.955) (width 2) (layer F.Cu) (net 1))
 (segment (start 38.735 22.225) (end 40.005 20.955) (width 2) (layer F.Cu) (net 1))
 (segment (start 55.245 22.225) (end 60.325 22.225) (width 2) (layer F.Cu) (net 1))
 (segment (start 60.325 22.225) (end 64.77 17.78) (width 2) (layer F.Cu) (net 1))
 (segment (start 64.77 17.78) (end 64.77 5.08) (width 2) (layer F.Cu) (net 1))
 (segment (start 62.865 3.175) (end 57.15 3.175) (width 2) (layer F.Cu) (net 1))
 (segment (start 64.77 5.08) (end 62.865 3.175) (width 2) (layer F.Cu) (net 1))
 (segment (start 55.245 35.56) (end 55.245 34.925) (width 0.25) (layer F.Cu) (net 1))
 (segment (start 51.435 39.37) (end 55.245 35.56) (width 2) (layer F.Cu) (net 1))
 (segment (start 55.245 34.925) (end 55.245 22.86) (width 2) (layer F.Cu) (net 1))
 (segment (start 46.355 24.13) (end 46.355 29.21) (width 2) (layer B.Cu) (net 2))
 (segment (start 46.355 29.21) (end 46.355 34.29) (width 2) (layer B.Cu) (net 2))
 (segment (start 46.355 34.29) (end 46.355 39.37) (width 2) (layer B.Cu) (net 2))
 (segment (start 46.355 44.45) (end 46.355 39.37) (width 2) (layer B.Cu) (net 2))
 (segment (start 46.355 24.13) (end 46.355 21.59) (width 2) (layer B.Cu) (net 2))
 (segment (start 46.355 21.59) (end 50.165 17.78) (width 2) (layer B.Cu) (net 2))
 (segment (start 50.165 17.78) (end 55.245 17.78) (width 2) (layer B.Cu) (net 2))
 (segment (start 57.15 15.875) (end 57.15 8.255) (width 2) (layer B.Cu) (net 2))
 (segment (start 55.245 17.78) (end 57.15 15.875) (width 2) (layer B.Cu) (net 2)))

